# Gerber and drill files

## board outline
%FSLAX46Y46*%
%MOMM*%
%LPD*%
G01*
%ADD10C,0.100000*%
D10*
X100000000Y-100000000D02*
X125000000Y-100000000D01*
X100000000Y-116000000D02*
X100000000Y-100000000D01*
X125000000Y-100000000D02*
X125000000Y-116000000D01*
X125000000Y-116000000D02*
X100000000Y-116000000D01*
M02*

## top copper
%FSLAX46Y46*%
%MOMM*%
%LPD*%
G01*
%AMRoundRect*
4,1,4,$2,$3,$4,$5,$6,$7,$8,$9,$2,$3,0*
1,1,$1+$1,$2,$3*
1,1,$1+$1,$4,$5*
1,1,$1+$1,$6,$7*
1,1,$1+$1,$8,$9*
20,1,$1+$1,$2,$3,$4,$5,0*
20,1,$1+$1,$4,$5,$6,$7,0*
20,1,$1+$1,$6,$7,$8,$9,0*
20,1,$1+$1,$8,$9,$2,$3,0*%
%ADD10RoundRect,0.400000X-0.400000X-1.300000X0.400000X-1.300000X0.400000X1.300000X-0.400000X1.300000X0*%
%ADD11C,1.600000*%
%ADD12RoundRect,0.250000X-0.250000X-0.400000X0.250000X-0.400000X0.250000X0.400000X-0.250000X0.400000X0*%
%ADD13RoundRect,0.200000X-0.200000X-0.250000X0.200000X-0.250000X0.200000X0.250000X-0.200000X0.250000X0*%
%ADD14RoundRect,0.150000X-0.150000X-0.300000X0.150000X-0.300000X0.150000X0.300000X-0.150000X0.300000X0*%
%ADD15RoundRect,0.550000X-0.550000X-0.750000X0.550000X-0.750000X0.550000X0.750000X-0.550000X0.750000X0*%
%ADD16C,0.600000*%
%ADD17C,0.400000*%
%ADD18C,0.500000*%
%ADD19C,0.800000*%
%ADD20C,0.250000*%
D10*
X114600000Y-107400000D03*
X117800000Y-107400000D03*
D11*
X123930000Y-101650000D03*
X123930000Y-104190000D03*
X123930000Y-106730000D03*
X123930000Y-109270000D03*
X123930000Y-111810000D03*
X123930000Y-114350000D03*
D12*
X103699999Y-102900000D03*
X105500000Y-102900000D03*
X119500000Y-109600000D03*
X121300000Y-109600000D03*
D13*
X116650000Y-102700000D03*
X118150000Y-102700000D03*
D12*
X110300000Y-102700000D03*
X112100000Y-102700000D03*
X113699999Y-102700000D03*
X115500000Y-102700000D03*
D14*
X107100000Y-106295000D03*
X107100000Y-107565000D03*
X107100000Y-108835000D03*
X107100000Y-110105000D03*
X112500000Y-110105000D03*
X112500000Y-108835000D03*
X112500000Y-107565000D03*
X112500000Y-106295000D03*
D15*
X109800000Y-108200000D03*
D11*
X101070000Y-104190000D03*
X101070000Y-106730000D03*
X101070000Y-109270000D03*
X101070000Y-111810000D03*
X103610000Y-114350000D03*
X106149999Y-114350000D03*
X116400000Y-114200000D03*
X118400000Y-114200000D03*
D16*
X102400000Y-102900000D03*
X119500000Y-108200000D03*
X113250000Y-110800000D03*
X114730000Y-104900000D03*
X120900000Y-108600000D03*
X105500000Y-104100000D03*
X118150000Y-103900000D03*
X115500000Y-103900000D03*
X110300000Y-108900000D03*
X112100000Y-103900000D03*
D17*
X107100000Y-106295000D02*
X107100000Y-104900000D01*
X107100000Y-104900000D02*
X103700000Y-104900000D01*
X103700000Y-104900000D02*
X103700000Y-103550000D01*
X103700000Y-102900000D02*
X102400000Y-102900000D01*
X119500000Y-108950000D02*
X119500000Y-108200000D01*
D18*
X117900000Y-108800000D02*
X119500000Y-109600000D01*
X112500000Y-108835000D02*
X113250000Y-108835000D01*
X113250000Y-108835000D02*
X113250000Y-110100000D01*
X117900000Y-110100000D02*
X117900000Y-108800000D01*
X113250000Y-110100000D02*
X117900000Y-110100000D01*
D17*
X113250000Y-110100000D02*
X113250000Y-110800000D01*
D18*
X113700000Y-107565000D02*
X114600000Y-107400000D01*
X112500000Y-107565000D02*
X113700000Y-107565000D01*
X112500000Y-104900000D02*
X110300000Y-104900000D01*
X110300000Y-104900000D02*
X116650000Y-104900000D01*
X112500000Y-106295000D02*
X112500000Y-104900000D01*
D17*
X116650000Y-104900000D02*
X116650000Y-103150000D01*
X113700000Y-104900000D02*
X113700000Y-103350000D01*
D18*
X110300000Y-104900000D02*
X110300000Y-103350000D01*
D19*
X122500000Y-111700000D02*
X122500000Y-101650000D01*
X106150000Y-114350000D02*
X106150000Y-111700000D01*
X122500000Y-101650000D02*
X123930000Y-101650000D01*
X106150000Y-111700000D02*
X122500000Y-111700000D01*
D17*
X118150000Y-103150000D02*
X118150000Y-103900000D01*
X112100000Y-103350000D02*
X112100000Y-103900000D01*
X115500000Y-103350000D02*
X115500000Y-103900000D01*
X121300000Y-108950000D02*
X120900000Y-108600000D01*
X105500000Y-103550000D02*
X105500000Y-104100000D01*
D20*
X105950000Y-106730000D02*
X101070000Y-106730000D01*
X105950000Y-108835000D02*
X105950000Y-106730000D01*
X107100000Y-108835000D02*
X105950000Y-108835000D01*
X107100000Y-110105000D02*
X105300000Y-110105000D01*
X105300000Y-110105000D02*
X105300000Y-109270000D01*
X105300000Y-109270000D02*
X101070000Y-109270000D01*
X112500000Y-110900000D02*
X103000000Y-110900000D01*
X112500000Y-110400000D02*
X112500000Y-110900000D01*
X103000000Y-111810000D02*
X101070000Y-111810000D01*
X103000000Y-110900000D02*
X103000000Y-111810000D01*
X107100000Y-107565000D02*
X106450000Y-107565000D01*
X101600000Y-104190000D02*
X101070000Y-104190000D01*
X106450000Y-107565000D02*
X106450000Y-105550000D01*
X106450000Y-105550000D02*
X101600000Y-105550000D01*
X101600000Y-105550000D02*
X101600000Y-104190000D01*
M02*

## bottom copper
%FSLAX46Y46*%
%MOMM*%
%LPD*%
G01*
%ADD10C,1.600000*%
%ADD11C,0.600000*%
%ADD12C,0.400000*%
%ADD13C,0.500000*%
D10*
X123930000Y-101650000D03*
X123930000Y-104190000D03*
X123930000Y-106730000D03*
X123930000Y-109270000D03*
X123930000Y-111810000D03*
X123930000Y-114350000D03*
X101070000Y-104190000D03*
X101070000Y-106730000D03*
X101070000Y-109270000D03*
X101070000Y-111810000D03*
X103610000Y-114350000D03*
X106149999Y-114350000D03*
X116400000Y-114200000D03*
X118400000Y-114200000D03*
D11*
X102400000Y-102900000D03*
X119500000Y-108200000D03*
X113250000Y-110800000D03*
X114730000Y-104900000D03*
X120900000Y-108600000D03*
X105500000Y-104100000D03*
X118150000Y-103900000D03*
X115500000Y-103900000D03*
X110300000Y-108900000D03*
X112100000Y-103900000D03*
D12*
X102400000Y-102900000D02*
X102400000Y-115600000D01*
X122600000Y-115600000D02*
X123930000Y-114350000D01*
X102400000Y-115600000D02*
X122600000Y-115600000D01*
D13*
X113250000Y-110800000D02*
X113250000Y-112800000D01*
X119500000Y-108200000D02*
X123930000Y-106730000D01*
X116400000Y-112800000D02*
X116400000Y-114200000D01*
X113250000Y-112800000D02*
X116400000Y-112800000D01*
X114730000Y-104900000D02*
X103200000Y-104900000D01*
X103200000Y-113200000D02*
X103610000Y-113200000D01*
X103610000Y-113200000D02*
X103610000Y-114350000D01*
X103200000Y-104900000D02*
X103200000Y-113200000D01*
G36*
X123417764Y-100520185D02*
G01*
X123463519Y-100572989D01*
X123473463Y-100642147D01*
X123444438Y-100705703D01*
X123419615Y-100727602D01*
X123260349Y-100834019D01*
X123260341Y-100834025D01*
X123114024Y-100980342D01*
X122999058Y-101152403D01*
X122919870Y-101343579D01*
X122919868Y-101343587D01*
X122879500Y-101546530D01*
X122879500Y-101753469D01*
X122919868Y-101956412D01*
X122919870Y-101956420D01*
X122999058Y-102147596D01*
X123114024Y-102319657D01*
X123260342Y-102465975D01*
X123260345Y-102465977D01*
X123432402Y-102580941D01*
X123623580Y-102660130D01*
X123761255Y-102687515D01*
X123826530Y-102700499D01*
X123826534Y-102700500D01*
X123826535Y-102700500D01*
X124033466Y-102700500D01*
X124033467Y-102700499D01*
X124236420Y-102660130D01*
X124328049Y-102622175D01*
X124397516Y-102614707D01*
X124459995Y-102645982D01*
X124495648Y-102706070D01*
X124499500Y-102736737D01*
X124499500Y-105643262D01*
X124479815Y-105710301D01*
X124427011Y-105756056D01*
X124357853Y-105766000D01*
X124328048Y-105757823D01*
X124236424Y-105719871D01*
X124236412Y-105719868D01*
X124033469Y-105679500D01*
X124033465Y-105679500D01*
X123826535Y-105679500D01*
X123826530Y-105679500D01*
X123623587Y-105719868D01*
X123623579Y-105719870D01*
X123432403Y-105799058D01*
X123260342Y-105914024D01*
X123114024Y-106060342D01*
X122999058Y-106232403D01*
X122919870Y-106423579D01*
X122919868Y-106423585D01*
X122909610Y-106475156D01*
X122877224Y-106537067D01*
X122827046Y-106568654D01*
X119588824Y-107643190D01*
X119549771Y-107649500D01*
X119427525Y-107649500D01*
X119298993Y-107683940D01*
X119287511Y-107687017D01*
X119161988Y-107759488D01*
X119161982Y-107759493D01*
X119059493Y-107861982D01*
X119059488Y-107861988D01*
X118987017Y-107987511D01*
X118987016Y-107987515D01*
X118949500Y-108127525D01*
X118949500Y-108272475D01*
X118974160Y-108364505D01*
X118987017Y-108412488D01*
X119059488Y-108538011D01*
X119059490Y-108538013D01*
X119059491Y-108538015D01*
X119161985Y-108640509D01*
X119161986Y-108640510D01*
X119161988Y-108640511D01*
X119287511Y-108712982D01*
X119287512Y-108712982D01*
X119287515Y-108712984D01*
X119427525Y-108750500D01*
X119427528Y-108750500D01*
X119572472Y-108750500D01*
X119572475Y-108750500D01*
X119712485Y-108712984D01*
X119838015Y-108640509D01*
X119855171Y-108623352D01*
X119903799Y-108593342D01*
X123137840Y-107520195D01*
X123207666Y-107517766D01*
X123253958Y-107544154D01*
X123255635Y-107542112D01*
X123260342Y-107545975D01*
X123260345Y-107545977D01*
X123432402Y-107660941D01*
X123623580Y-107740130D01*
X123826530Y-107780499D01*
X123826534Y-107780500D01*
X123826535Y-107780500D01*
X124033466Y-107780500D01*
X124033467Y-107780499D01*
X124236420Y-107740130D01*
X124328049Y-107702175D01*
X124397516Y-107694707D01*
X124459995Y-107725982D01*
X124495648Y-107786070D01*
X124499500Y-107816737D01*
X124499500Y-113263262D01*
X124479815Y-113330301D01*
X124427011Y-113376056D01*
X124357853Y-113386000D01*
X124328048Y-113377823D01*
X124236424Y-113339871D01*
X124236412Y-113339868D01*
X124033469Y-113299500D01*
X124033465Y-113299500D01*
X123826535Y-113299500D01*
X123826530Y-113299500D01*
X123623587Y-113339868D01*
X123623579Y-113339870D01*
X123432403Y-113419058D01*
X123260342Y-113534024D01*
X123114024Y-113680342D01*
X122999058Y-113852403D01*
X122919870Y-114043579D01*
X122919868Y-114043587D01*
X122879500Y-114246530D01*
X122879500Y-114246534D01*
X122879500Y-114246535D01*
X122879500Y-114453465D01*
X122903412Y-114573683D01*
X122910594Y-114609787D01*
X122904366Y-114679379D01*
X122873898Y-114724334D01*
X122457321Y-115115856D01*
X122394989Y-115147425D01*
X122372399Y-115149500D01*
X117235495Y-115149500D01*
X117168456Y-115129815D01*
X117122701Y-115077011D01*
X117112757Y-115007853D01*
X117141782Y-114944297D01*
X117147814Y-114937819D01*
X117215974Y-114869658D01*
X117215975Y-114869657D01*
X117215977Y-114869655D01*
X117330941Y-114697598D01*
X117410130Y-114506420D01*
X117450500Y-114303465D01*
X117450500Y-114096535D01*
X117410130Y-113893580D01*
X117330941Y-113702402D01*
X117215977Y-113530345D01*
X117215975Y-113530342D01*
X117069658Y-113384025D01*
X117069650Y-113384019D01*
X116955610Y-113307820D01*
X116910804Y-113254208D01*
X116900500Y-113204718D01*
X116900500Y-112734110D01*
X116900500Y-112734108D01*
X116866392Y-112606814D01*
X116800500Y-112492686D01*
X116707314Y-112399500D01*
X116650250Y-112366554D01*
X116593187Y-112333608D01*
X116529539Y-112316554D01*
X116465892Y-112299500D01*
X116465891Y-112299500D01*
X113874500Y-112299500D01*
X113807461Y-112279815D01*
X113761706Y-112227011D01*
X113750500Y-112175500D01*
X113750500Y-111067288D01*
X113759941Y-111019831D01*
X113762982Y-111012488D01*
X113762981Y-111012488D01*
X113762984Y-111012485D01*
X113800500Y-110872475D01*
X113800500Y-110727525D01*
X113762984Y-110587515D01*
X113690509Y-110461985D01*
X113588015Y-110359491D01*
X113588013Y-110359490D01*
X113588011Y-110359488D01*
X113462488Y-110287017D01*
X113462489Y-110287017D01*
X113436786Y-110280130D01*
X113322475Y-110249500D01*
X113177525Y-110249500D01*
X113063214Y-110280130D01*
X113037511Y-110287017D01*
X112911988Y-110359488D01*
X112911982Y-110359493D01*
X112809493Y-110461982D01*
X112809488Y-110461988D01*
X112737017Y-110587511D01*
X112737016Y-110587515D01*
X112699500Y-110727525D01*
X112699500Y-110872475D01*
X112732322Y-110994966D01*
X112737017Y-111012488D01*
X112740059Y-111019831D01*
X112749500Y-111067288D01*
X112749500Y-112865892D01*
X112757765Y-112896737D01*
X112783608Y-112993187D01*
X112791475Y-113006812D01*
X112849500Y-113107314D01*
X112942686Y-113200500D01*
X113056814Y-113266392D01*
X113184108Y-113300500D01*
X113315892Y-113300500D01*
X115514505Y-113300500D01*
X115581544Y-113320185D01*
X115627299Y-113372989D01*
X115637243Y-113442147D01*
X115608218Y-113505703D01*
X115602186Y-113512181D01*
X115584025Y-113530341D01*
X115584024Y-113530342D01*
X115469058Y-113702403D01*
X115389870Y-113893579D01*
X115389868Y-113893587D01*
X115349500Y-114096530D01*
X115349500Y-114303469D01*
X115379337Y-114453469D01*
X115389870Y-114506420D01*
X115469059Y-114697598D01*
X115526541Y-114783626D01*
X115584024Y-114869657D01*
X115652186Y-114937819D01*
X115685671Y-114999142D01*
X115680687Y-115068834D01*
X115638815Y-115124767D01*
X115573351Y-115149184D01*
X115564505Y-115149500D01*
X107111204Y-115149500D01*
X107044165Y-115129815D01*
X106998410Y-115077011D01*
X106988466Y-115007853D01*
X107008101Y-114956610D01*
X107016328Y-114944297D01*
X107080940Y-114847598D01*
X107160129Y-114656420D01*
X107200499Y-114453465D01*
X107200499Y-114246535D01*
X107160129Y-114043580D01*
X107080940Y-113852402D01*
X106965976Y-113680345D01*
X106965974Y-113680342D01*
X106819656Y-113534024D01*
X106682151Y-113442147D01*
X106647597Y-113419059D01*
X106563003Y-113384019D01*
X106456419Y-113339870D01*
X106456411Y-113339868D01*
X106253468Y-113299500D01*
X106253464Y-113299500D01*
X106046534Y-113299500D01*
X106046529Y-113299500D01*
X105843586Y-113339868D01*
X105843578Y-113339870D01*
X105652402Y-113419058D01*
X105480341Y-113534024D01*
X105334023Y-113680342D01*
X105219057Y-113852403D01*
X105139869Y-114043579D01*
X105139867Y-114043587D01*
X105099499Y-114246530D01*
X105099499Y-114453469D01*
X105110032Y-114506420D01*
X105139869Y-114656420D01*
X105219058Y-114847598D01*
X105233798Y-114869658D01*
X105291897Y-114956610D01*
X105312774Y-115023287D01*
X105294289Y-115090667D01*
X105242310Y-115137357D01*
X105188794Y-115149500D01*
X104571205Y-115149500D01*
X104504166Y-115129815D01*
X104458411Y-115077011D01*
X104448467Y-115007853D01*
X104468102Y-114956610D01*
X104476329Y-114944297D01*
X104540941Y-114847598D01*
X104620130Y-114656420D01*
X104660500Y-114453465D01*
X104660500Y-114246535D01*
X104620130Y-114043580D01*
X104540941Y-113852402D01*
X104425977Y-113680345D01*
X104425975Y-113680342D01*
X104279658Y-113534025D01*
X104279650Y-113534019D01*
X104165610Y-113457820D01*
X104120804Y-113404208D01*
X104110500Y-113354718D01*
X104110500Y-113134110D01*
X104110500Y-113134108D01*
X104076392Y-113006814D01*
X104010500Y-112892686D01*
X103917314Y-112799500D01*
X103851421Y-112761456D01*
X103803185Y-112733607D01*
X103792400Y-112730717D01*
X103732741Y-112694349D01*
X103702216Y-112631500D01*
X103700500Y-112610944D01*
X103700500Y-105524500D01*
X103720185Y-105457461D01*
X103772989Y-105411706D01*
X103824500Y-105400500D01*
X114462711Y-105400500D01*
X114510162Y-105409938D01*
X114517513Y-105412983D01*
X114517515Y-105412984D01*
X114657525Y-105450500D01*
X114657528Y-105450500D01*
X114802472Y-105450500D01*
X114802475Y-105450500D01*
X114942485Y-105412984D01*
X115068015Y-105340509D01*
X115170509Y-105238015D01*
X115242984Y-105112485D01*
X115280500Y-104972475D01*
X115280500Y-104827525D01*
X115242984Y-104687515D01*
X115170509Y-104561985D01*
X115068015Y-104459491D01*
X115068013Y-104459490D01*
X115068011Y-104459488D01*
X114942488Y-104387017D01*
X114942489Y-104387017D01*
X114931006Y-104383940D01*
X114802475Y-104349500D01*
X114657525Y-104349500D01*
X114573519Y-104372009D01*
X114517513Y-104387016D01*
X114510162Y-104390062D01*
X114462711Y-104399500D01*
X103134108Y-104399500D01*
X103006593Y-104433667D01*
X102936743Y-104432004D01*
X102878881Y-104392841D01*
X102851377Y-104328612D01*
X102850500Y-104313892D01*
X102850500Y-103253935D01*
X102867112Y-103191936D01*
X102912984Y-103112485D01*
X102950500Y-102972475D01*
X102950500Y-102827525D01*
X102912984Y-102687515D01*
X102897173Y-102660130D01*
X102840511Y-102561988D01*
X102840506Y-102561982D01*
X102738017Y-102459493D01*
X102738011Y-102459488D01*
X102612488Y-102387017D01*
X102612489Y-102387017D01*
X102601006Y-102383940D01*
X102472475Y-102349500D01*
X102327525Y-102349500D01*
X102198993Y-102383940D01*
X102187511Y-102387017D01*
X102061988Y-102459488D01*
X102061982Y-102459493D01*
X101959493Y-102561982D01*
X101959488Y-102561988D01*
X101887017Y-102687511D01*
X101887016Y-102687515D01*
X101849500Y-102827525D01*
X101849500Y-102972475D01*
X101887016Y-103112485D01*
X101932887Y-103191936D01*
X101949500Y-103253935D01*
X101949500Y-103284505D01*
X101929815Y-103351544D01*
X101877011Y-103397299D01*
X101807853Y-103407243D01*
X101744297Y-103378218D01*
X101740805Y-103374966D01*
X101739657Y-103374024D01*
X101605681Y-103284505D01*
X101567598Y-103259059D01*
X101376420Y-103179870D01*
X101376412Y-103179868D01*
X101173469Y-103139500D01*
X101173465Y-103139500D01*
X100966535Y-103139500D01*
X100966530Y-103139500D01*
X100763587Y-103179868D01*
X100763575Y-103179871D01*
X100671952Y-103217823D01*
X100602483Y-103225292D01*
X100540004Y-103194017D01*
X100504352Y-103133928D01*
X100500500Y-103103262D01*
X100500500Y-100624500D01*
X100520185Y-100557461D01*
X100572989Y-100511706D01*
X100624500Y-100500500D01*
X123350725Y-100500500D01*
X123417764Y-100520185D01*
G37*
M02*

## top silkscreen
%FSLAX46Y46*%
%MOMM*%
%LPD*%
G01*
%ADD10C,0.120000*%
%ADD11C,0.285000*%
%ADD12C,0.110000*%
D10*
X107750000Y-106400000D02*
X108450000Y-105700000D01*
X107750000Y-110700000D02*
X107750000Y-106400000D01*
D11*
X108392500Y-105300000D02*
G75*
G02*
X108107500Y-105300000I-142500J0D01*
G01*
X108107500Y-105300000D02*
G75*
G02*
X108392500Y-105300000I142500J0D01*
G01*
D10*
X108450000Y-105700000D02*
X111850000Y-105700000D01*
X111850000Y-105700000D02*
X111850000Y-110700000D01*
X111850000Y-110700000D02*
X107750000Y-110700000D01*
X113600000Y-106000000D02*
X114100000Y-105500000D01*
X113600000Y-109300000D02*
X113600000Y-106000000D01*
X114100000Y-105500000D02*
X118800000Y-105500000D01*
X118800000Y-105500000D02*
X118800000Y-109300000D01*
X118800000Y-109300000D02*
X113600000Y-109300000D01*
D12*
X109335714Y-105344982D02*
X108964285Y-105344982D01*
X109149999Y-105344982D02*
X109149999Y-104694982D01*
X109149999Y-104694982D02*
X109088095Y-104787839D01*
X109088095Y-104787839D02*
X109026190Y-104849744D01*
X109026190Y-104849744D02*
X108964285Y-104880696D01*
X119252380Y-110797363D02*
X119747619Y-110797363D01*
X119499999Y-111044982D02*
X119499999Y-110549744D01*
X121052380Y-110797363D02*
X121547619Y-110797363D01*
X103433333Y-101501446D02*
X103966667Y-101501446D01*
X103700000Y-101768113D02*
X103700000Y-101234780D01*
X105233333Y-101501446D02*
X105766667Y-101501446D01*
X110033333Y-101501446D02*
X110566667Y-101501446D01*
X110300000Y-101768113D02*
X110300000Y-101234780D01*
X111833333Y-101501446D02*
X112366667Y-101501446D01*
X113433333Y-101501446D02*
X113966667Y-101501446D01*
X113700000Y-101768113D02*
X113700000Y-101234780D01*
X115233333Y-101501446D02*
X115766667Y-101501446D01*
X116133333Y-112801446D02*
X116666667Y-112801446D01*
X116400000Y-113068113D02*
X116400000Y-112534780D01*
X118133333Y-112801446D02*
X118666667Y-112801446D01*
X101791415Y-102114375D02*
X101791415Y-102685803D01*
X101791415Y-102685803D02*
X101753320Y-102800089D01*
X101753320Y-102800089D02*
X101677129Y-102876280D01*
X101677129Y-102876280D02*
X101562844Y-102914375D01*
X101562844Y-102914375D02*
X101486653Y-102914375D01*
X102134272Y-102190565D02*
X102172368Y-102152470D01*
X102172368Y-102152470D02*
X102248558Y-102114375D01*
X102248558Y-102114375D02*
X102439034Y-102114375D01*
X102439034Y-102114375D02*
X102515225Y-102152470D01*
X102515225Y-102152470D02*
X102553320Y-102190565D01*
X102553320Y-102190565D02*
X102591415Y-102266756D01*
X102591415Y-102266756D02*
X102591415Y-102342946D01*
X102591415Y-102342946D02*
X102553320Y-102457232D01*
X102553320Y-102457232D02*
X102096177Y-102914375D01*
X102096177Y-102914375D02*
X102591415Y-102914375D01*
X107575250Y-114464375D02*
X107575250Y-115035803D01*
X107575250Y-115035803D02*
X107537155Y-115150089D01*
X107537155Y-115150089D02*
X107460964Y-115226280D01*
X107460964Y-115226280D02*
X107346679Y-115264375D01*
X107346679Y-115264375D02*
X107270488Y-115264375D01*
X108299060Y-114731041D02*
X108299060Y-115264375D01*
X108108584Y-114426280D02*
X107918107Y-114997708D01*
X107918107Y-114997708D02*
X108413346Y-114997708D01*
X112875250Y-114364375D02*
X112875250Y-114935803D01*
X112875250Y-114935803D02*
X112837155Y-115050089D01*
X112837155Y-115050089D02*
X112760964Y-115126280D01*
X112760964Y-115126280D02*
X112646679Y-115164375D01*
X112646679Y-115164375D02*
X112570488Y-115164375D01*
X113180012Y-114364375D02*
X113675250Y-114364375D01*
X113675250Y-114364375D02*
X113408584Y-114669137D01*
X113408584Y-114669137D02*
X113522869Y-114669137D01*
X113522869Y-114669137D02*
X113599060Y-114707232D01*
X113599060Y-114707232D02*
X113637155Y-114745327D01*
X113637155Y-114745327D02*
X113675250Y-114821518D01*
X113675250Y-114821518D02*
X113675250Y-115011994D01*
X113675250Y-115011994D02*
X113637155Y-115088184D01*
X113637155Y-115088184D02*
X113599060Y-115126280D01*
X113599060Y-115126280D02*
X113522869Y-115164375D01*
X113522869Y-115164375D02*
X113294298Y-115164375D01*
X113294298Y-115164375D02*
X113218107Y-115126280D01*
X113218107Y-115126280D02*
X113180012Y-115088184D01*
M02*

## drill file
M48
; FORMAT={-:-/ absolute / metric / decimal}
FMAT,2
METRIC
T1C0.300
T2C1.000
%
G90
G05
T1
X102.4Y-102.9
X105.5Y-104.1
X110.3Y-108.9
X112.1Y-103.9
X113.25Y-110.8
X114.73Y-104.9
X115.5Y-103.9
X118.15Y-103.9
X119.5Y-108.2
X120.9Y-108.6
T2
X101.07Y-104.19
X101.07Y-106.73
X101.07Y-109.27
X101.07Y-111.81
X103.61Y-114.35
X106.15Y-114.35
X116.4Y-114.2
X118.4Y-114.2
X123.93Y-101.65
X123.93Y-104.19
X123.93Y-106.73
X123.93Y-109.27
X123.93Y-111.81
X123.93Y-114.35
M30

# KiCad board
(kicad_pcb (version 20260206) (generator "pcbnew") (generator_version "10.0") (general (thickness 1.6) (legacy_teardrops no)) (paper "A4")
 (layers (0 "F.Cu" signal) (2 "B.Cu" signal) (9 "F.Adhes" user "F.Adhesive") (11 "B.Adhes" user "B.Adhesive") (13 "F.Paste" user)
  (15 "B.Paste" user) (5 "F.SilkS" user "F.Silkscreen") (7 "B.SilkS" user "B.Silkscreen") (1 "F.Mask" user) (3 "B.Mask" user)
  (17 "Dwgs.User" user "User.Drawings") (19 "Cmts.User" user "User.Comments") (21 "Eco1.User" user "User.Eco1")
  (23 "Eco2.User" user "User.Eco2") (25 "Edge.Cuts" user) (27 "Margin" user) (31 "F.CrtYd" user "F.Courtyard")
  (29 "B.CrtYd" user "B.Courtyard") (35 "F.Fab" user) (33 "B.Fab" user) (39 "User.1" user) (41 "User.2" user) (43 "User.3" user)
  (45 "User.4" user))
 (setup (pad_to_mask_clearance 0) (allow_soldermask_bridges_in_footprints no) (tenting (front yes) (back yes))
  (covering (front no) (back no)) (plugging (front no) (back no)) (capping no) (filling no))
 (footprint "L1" (layer "F.Cu") (at 116.2 107.4)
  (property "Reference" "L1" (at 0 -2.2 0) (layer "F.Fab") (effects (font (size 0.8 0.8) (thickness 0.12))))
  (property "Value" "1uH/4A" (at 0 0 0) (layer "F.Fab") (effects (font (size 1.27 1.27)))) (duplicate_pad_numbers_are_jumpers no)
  (pad "1" smd roundrect (at -1.6 0) (size 1.6 3.4) (layers "F.Cu" "F.Mask" "F.Paste") (roundrect_rratio 0.25) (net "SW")
   (thermal_bridge_angle 45))
  (pad "2" smd roundrect (at 1.6 0) (size 1.6 3.4) (layers "F.Cu" "F.Mask" "F.Paste") (roundrect_rratio 0.25) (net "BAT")
   (thermal_bridge_angle 45)))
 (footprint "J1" (layer "F.Cu") (at 123.93 108)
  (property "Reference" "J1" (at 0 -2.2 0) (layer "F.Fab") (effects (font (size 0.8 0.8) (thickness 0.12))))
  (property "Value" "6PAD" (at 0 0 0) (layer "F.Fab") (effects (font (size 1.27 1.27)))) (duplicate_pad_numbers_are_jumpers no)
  (pad "1" thru_hole circle (at 0 -6.35) (size 1.6 1.6) (drill 1) (layers "*.Cu" "*.Mask") (remove_unused_layers no) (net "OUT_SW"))
  (pad "2" thru_hole circle (at 0 -3.81) (size 1.6 1.6) (drill 1) (layers "*.Cu" "*.Mask") (remove_unused_layers no) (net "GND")
   (zone_connect 2))
  (pad "3" thru_hole circle (at 0 -1.27) (size 1.6 1.6) (drill 1) (layers "*.Cu" "*.Mask") (remove_unused_layers no) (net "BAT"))
  (pad "4" thru_hole circle (at 0 1.27) (size 1.6 1.6) (drill 1) (layers "*.Cu" "*.Mask") (remove_unused_layers no) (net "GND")
   (zone_connect 2))
  (pad "5" thru_hole circle (at 0 3.81) (size 1.6 1.6) (drill 1) (layers "*.Cu" "*.Mask") (remove_unused_layers no) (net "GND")
   (zone_connect 2))
  (pad "6" thru_hole circle (at 0 6.35) (size 1.6 1.6) (drill 1) (layers "*.Cu" "*.Mask") (remove_unused_layers no) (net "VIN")))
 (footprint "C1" (layer "F.Cu") (at 104.6 102.9)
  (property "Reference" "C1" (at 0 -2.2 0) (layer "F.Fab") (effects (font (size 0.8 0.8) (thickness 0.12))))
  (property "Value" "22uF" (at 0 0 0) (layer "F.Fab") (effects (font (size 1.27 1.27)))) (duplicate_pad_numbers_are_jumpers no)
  (pad "1" smd roundrect (at -0.900001 0) (size 1 1.3) (layers "F.Cu" "F.Mask" "F.Paste") (roundrect_rratio 0.25) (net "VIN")
   (thermal_bridge_angle 45))
  (pad "2" smd roundrect (at 0.9 0) (size 1 1.3) (layers "F.Cu" "F.Mask" "F.Paste") (roundrect_rratio 0.25) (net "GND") (zone_connect 2)
   (thermal_bridge_angle 45)))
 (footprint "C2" (layer "F.Cu") (at 120.4 109.6)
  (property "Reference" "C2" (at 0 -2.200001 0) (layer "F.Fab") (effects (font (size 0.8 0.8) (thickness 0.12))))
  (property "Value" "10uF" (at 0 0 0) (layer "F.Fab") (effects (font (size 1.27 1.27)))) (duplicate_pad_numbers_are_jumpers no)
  (pad "1" smd roundrect (at -0.9 0) (size 1 1.3) (layers "F.Cu" "F.Mask" "F.Paste") (roundrect_rratio 0.25) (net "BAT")
   (thermal_bridge_angle 45))
  (pad "2" smd roundrect (at 0.9 0) (size 1 1.3) (layers "F.Cu" "F.Mask" "F.Paste") (roundrect_rratio 0.25) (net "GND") (zone_connect 2)
   (thermal_bridge_angle 45)))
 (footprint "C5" (layer "F.Cu") (at 117.4 102.7)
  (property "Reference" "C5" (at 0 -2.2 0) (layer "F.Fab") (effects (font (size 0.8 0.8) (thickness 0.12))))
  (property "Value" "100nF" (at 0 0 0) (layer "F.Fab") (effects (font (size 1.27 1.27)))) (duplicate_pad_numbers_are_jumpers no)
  (pad "1" smd roundrect (at -0.75 0) (size 0.8 0.9) (layers "F.Cu" "F.Mask" "F.Paste") (roundrect_rratio 0.25) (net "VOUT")
   (thermal_bridge_angle 45))
  (pad "2" smd roundrect (at 0.75 0) (size 0.8 0.9) (layers "F.Cu" "F.Mask" "F.Paste") (roundrect_rratio 0.25) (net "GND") (zone_connect 2)
   (thermal_bridge_angle 45)))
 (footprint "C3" (layer "F.Cu") (at 111.2 102.7)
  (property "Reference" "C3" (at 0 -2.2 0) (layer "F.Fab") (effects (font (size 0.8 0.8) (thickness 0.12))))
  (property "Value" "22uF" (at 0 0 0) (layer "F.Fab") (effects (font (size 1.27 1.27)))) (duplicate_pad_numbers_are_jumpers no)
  (pad "1" smd roundrect (at -0.9 0) (size 1 1.3) (layers "F.Cu" "F.Mask" "F.Paste") (roundrect_rratio 0.25) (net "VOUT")
   (thermal_bridge_angle 45))
  (pad "2" smd roundrect (at 0.9 0) (size 1 1.3) (layers "F.Cu" "F.Mask" "F.Paste") (roundrect_rratio 0.25) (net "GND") (zone_connect 2)
   (thermal_bridge_angle 45)))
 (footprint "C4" (layer "F.Cu") (at 114.6 102.7)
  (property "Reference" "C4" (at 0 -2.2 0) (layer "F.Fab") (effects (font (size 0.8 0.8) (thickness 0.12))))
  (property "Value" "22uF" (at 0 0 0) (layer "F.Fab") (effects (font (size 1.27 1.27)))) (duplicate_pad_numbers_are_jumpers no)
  (pad "1" smd roundrect (at -0.900001 0) (size 1 1.3) (layers "F.Cu" "F.Mask" "F.Paste") (roundrect_rratio 0.25) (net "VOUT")
   (thermal_bridge_angle 45))
  (pad "2" smd roundrect (at 0.9 0) (size 1 1.3) (layers "F.Cu" "F.Mask" "F.Paste") (roundrect_rratio 0.25) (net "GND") (zone_connect 2)
   (thermal_bridge_angle 45)))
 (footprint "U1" (layer "F.Cu") (at 109.8 108.2)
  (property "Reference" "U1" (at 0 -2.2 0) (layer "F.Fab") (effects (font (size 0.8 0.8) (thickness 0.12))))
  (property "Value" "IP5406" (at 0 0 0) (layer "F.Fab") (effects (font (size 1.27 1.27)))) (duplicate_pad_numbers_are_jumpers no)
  (pad "1" smd roundrect (at -2.7 -1.905) (size 0.6 0.9) (layers "F.Cu" "F.Mask" "F.Paste") (roundrect_rratio 0.25) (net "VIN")
   (thermal_bridge_angle 45))
  (pad "2" smd roundrect (at -2.7 -0.635) (size 0.6 0.9) (layers "F.Cu" "F.Mask" "F.Paste") (roundrect_rratio 0.25) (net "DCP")
   (thermal_bridge_angle 45))
  (pad "3" smd roundrect (at -2.7 0.635) (size 0.6 0.9) (layers "F.Cu" "F.Mask" "F.Paste") (roundrect_rratio 0.25) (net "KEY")
   (thermal_bridge_angle 45))
  (pad "4" smd roundrect (at -2.7 1.905) (size 0.6 0.9) (layers "F.Cu" "F.Mask" "F.Paste") (roundrect_rratio 0.25) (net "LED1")
   (thermal_bridge_angle 45))
  (pad "5" smd roundrect (at 2.7 1.905) (size 0.6 0.9) (layers "F.Cu" "F.Mask" "F.Paste") (roundrect_rratio 0.25) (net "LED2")
   (thermal_bridge_angle 45))
  (pad "6" smd roundrect (at 2.7 0.635) (size 0.6 0.9) (layers "F.Cu" "F.Mask" "F.Paste") (roundrect_rratio 0.25) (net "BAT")
   (thermal_bridge_angle 45))
  (pad "7" smd roundrect (at 2.7 -0.635) (size 0.6 0.9) (layers "F.Cu" "F.Mask" "F.Paste") (roundrect_rratio 0.25) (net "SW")
   (thermal_bridge_angle 45))
  (pad "8" smd roundrect (at 2.7 -1.905) (size 0.6 0.9) (layers "F.Cu" "F.Mask" "F.Paste") (roundrect_rratio 0.25) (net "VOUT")
   (thermal_bridge_angle 45))
  (pad "9" smd roundrect (at 0 0) (size 2.2 2.6) (layers "F.Cu" "F.Mask" "F.Paste") (roundrect_rratio 0.25) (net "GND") (zone_connect 2)
   (thermal_bridge_angle 45)))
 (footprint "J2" (layer "F.Cu") (at 101.07 108)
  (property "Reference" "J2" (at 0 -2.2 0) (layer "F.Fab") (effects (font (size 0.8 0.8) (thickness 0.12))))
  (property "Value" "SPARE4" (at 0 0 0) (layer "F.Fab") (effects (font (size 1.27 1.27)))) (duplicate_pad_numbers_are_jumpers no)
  (pad "1" thru_hole circle (at 0 -3.81) (size 1.6 1.6) (drill 1) (layers "*.Cu" "*.Mask") (remove_unused_layers no) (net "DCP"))
  (pad "2" thru_hole circle (at 0 -1.27) (size 1.6 1.6) (drill 1) (layers "*.Cu" "*.Mask") (remove_unused_layers no) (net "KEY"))
  (pad "3" thru_hole circle (at 0 1.27) (size 1.6 1.6) (drill 1) (layers "*.Cu" "*.Mask") (remove_unused_layers no) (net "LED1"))
  (pad "4" thru_hole circle (at 0 3.81) (size 1.6 1.6) (drill 1) (layers "*.Cu" "*.Mask") (remove_unused_layers no) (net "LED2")))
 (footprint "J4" (layer "F.Cu") (at 104.88 114.35)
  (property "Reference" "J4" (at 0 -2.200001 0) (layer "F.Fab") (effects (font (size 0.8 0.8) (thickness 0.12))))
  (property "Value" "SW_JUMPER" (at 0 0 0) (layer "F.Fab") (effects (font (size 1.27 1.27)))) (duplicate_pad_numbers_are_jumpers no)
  (pad "1" thru_hole circle (at -1.27 0) (size 1.6 1.6) (drill 1) (layers "*.Cu" "*.Mask") (remove_unused_layers no) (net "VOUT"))
  (pad "2" thru_hole circle (at 1.269999 0) (size 1.6 1.6) (drill 1) (layers "*.Cu" "*.Mask") (remove_unused_layers no) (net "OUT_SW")))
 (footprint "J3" (layer "F.Cu") (at 117.4 114.2)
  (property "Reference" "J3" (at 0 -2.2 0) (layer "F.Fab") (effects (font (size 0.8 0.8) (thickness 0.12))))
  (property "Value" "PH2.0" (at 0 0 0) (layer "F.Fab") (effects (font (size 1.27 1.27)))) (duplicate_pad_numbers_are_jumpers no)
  (pad "1" thru_hole circle (at -1 0) (size 1.6 1.6) (drill 1) (layers "*.Cu" "*.Mask") (remove_unused_layers no) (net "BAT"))
  (pad "2" thru_hole circle (at 1 0) (size 1.6 1.6) (drill 1) (layers "*.Cu" "*.Mask") (remove_unused_layers no) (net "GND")
   (zone_connect 2)))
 (gr_line (start 107.75 106.4) (end 108.45 105.7) (stroke (width 0.12) (type default)) (layer "F.SilkS"))
 (gr_line (start 107.75 110.7) (end 107.75 106.4) (stroke (width 0.12) (type default)) (layer "F.SilkS"))
 (gr_circle (center 108.25 105.3) (end 108.53 105.3) (stroke (width 0.01) (type default)) (fill yes) (layer "F.SilkS"))
 (gr_line (start 108.45 105.7) (end 111.85 105.7) (stroke (width 0.12) (type default)) (layer "F.SilkS"))
 (gr_line (start 111.85 105.7) (end 111.85 110.7) (stroke (width 0.12) (type default)) (layer "F.SilkS"))
 (gr_line (start 111.85 110.7) (end 107.75 110.7) (stroke (width 0.12) (type default)) (layer "F.SilkS"))
 (gr_line (start 113.6 106) (end 114.1 105.5) (stroke (width 0.12) (type default)) (layer "F.SilkS"))
 (gr_line (start 113.6 109.3) (end 113.6 106) (stroke (width 0.12) (type default)) (layer "F.SilkS"))
 (gr_line (start 114.1 105.5) (end 118.8 105.5) (stroke (width 0.12) (type default)) (layer "F.SilkS"))
 (gr_line (start 118.8 105.5) (end 118.8 109.3) (stroke (width 0.12) (type default)) (layer "F.SilkS"))
 (gr_line (start 118.8 109.3) (end 113.6 109.3) (stroke (width 0.12) (type default)) (layer "F.SilkS"))
 (gr_line (start 100 100) (end 125 100) (stroke (width 0.1) (type default)) (layer "Edge.Cuts"))
 (gr_line (start 100 116) (end 100 100) (stroke (width 0.1) (type default)) (layer "Edge.Cuts"))
 (gr_line (start 125 100) (end 125 116) (stroke (width 0.1) (type default)) (layer "Edge.Cuts"))
 (gr_line (start 125 116) (end 100 116) (stroke (width 0.1) (type default)) (layer "Edge.Cuts"))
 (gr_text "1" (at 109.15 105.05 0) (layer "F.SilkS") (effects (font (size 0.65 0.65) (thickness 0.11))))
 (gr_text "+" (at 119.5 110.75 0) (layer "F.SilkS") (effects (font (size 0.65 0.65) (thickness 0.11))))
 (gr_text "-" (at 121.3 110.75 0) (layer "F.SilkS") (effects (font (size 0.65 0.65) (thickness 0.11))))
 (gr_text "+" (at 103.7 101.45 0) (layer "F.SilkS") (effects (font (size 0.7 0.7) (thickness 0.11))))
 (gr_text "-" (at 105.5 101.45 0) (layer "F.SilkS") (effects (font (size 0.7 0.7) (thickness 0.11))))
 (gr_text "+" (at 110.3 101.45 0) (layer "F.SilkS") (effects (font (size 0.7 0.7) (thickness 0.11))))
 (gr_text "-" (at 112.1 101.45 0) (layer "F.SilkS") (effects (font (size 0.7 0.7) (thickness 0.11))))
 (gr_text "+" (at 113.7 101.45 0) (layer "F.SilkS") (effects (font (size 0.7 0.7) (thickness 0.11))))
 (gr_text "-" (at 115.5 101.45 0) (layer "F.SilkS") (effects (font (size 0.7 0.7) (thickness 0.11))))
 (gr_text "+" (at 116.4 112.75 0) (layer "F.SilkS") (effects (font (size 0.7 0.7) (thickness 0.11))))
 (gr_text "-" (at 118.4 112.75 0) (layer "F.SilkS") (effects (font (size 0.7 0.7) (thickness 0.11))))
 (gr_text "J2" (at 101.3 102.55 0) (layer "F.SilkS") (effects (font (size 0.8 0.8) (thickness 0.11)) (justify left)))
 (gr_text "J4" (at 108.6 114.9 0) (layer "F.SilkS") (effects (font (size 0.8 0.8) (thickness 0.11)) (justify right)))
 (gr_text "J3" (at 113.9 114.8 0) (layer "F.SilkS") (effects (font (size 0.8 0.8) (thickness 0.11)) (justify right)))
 (segment (start 107.1 106.295) (end 107.1 104.9) (width 0.4) (layer "F.Cu") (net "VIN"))
 (segment (start 107.1 104.9) (end 103.7 104.9) (width 0.4) (layer "F.Cu") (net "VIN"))
 (segment (start 103.7 104.9) (end 103.7 103.55) (width 0.4) (layer "F.Cu") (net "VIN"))
 (segment (start 103.7 102.9) (end 102.4 102.9) (width 0.4) (layer "F.Cu") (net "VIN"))
 (via (at 102.4 102.9) (size 0.6) (drill 0.3) (layers "F.Cu" "B.Cu") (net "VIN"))
 (segment (start 102.4 102.9) (end 102.4 115.6) (width 0.4) (layer "B.Cu") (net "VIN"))
 (segment (start 122.6 115.6) (end 123.93 114.35) (width 0.4) (layer "B.Cu") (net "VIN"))
 (segment (start 102.4 115.6) (end 122.6 115.6) (width 0.4) (layer "B.Cu") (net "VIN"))
 (segment (start 119.5 108.95) (end 119.5 108.2) (width 0.4) (layer "F.Cu") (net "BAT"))
 (segment (start 117.9 108.8) (end 119.5 109.6) (width 0.5) (layer "F.Cu") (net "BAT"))
 (segment (start 112.5 108.835) (end 113.25 108.835) (width 0.5) (layer "F.Cu") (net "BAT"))
 (segment (start 113.25 108.835) (end 113.25 110.1) (width 0.5) (layer "F.Cu") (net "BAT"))
 (segment (start 117.9 110.1) (end 117.9 108.8) (width 0.5) (layer "F.Cu") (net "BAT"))
 (segment (start 113.25 110.1) (end 117.9 110.1) (width 0.5) (layer "F.Cu") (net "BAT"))
 (segment (start 113.25 110.1) (end 113.25 110.8) (width 0.4) (layer "F.Cu") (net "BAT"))
 (via (at 119.5 108.2) (size 0.6) (drill 0.3) (layers "F.Cu" "B.Cu") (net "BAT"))
 (via (at 113.25 110.8) (size 0.6) (drill 0.3) (layers "F.Cu" "B.Cu") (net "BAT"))
 (segment (start 113.25 110.8) (end 113.25 112.8) (width 0.5) (layer "B.Cu") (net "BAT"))
 (segment (start 119.5 108.2) (end 123.93 106.73) (width 0.5) (layer "B.Cu") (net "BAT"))
 (segment (start 116.4 112.8) (end 116.4 114.2) (width 0.5) (layer "B.Cu") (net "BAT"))
 (segment (start 113.25 112.8) (end 116.4 112.8) (width 0.5) (layer "B.Cu") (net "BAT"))
 (segment (start 113.7 107.565) (end 114.6 107.4) (width 0.5) (layer "F.Cu") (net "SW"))
 (segment (start 112.5 107.565) (end 113.7 107.565) (width 0.5) (layer "F.Cu") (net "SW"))
 (segment (start 112.5 104.9) (end 110.3 104.9) (width 0.5) (layer "F.Cu") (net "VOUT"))
 (segment (start 110.3 104.9) (end 116.65 104.9) (width 0.5) (layer "F.Cu") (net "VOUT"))
 (segment (start 112.5 106.295) (end 112.5 104.9) (width 0.5) (layer "F.Cu") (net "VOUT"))
 (segment (start 116.65 104.9) (end 116.65 103.15) (width 0.4) (layer "F.Cu") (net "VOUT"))
 (segment (start 113.7 104.9) (end 113.7 103.35) (width 0.4) (layer "F.Cu") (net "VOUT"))
 (segment (start 110.3 104.9) (end 110.3 103.35) (width 0.5) (layer "F.Cu") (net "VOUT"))
 (via (at 114.73 104.9) (size 0.6) (drill 0.3) (layers "F.Cu" "B.Cu") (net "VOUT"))
 (segment (start 114.73 104.9) (end 103.2 104.9) (width 0.5) (layer "B.Cu") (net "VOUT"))
 (segment (start 103.2 113.2) (end 103.61 113.2) (width 0.5) (layer "B.Cu") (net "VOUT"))
 (segment (start 103.61 113.2) (end 103.61 114.35) (width 0.5) (layer "B.Cu") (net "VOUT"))
 (segment (start 103.2 104.9) (end 103.2 113.2) (width 0.5) (layer "B.Cu") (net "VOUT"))
 (segment (start 122.5 111.7) (end 122.5 101.65) (width 0.8) (layer "F.Cu") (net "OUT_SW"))
 (segment (start 106.15 114.35) (end 106.15 111.7) (width 0.8) (layer "F.Cu") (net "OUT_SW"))
 (segment (start 122.5 101.65) (end 123.93 101.65) (width 0.8) (layer "F.Cu") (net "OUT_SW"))
 (segment (start 106.15 111.7) (end 122.5 111.7) (width 0.8) (layer "F.Cu") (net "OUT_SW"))
 (segment (start 118.15 103.15) (end 118.15 103.9) (width 0.4) (layer "F.Cu") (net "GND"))
 (segment (start 112.1 103.35) (end 112.1 103.9) (width 0.4) (layer "F.Cu") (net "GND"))
 (segment (start 115.5 103.35) (end 115.5 103.9) (width 0.4) (layer "F.Cu") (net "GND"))
 (segment (start 121.3 108.95) (end 120.9 108.6) (width 0.4) (layer "F.Cu") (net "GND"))
 (segment (start 105.5 103.55) (end 105.5 104.1) (width 0.4) (layer "F.Cu") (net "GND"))
 (via (at 120.9 108.6) (size 0.6) (drill 0.3) (layers "F.Cu" "B.Cu") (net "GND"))
 (via (at 105.5 104.1) (size 0.6) (drill 0.3) (layers "F.Cu" "B.Cu") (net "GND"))
 (via (at 118.15 103.9) (size 0.6) (drill 0.3) (layers "F.Cu" "B.Cu") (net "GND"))
 (via (at 115.5 103.9) (size 0.6) (drill 0.3) (layers "F.Cu" "B.Cu") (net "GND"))
 (via (at 110.3 108.9) (size 0.6) (drill 0.3) (layers "F.Cu" "B.Cu") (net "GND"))
 (via (at 112.1 103.9) (size 0.6) (drill 0.3) (layers "F.Cu" "B.Cu") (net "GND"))
 (segment (start 105.95 106.73) (end 101.07 106.73) (width 0.25) (layer "F.Cu") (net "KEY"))
 (segment (start 105.95 108.835) (end 105.95 106.73) (width 0.25) (layer "F.Cu") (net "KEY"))
 (segment (start 107.1 108.835) (end 105.95 108.835) (width 0.25) (layer "F.Cu") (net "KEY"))
 (segment (start 107.1 110.105) (end 105.3 110.105) (width 0.25) (layer "F.Cu") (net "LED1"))
 (segment (start 105.3 110.105) (end 105.3 109.27) (width 0.25) (layer "F.Cu") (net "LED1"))
 (segment (start 105.3 109.27) (end 101.07 109.27) (width 0.25) (layer "F.Cu") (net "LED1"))
 (segment (start 112.5 110.9) (end 103 110.9) (width 0.25) (layer "F.Cu") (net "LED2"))
 (segment (start 112.5 110.4) (end 112.5 110.9) (width 0.25) (layer "F.Cu") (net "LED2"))
 (segment (start 103 111.81) (end 101.07 111.81) (width 0.25) (layer "F.Cu") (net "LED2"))
 (segment (start 103 110.9) (end 103 111.81) (width 0.25) (layer "F.Cu") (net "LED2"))
 (segment (start 107.1 107.565) (end 106.45 107.565) (width 0.25) (layer "F.Cu") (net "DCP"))
 (segment (start 101.6 104.19) (end 101.07 104.19) (width 0.25) (layer "F.Cu") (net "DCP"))
 (segment (start 106.45 107.565) (end 106.45 105.55) (width 0.25) (layer "F.Cu") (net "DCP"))
 (segment (start 106.45 105.55) (end 101.6 105.55) (width 0.25) (layer "F.Cu") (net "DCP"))
 (segment (start 101.6 105.55) (end 101.6 104.19) (width 0.25) (layer "F.Cu") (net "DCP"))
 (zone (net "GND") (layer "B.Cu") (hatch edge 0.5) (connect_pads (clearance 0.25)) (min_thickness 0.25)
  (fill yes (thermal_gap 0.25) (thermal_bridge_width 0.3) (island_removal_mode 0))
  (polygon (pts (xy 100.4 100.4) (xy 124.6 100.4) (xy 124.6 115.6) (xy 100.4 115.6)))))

